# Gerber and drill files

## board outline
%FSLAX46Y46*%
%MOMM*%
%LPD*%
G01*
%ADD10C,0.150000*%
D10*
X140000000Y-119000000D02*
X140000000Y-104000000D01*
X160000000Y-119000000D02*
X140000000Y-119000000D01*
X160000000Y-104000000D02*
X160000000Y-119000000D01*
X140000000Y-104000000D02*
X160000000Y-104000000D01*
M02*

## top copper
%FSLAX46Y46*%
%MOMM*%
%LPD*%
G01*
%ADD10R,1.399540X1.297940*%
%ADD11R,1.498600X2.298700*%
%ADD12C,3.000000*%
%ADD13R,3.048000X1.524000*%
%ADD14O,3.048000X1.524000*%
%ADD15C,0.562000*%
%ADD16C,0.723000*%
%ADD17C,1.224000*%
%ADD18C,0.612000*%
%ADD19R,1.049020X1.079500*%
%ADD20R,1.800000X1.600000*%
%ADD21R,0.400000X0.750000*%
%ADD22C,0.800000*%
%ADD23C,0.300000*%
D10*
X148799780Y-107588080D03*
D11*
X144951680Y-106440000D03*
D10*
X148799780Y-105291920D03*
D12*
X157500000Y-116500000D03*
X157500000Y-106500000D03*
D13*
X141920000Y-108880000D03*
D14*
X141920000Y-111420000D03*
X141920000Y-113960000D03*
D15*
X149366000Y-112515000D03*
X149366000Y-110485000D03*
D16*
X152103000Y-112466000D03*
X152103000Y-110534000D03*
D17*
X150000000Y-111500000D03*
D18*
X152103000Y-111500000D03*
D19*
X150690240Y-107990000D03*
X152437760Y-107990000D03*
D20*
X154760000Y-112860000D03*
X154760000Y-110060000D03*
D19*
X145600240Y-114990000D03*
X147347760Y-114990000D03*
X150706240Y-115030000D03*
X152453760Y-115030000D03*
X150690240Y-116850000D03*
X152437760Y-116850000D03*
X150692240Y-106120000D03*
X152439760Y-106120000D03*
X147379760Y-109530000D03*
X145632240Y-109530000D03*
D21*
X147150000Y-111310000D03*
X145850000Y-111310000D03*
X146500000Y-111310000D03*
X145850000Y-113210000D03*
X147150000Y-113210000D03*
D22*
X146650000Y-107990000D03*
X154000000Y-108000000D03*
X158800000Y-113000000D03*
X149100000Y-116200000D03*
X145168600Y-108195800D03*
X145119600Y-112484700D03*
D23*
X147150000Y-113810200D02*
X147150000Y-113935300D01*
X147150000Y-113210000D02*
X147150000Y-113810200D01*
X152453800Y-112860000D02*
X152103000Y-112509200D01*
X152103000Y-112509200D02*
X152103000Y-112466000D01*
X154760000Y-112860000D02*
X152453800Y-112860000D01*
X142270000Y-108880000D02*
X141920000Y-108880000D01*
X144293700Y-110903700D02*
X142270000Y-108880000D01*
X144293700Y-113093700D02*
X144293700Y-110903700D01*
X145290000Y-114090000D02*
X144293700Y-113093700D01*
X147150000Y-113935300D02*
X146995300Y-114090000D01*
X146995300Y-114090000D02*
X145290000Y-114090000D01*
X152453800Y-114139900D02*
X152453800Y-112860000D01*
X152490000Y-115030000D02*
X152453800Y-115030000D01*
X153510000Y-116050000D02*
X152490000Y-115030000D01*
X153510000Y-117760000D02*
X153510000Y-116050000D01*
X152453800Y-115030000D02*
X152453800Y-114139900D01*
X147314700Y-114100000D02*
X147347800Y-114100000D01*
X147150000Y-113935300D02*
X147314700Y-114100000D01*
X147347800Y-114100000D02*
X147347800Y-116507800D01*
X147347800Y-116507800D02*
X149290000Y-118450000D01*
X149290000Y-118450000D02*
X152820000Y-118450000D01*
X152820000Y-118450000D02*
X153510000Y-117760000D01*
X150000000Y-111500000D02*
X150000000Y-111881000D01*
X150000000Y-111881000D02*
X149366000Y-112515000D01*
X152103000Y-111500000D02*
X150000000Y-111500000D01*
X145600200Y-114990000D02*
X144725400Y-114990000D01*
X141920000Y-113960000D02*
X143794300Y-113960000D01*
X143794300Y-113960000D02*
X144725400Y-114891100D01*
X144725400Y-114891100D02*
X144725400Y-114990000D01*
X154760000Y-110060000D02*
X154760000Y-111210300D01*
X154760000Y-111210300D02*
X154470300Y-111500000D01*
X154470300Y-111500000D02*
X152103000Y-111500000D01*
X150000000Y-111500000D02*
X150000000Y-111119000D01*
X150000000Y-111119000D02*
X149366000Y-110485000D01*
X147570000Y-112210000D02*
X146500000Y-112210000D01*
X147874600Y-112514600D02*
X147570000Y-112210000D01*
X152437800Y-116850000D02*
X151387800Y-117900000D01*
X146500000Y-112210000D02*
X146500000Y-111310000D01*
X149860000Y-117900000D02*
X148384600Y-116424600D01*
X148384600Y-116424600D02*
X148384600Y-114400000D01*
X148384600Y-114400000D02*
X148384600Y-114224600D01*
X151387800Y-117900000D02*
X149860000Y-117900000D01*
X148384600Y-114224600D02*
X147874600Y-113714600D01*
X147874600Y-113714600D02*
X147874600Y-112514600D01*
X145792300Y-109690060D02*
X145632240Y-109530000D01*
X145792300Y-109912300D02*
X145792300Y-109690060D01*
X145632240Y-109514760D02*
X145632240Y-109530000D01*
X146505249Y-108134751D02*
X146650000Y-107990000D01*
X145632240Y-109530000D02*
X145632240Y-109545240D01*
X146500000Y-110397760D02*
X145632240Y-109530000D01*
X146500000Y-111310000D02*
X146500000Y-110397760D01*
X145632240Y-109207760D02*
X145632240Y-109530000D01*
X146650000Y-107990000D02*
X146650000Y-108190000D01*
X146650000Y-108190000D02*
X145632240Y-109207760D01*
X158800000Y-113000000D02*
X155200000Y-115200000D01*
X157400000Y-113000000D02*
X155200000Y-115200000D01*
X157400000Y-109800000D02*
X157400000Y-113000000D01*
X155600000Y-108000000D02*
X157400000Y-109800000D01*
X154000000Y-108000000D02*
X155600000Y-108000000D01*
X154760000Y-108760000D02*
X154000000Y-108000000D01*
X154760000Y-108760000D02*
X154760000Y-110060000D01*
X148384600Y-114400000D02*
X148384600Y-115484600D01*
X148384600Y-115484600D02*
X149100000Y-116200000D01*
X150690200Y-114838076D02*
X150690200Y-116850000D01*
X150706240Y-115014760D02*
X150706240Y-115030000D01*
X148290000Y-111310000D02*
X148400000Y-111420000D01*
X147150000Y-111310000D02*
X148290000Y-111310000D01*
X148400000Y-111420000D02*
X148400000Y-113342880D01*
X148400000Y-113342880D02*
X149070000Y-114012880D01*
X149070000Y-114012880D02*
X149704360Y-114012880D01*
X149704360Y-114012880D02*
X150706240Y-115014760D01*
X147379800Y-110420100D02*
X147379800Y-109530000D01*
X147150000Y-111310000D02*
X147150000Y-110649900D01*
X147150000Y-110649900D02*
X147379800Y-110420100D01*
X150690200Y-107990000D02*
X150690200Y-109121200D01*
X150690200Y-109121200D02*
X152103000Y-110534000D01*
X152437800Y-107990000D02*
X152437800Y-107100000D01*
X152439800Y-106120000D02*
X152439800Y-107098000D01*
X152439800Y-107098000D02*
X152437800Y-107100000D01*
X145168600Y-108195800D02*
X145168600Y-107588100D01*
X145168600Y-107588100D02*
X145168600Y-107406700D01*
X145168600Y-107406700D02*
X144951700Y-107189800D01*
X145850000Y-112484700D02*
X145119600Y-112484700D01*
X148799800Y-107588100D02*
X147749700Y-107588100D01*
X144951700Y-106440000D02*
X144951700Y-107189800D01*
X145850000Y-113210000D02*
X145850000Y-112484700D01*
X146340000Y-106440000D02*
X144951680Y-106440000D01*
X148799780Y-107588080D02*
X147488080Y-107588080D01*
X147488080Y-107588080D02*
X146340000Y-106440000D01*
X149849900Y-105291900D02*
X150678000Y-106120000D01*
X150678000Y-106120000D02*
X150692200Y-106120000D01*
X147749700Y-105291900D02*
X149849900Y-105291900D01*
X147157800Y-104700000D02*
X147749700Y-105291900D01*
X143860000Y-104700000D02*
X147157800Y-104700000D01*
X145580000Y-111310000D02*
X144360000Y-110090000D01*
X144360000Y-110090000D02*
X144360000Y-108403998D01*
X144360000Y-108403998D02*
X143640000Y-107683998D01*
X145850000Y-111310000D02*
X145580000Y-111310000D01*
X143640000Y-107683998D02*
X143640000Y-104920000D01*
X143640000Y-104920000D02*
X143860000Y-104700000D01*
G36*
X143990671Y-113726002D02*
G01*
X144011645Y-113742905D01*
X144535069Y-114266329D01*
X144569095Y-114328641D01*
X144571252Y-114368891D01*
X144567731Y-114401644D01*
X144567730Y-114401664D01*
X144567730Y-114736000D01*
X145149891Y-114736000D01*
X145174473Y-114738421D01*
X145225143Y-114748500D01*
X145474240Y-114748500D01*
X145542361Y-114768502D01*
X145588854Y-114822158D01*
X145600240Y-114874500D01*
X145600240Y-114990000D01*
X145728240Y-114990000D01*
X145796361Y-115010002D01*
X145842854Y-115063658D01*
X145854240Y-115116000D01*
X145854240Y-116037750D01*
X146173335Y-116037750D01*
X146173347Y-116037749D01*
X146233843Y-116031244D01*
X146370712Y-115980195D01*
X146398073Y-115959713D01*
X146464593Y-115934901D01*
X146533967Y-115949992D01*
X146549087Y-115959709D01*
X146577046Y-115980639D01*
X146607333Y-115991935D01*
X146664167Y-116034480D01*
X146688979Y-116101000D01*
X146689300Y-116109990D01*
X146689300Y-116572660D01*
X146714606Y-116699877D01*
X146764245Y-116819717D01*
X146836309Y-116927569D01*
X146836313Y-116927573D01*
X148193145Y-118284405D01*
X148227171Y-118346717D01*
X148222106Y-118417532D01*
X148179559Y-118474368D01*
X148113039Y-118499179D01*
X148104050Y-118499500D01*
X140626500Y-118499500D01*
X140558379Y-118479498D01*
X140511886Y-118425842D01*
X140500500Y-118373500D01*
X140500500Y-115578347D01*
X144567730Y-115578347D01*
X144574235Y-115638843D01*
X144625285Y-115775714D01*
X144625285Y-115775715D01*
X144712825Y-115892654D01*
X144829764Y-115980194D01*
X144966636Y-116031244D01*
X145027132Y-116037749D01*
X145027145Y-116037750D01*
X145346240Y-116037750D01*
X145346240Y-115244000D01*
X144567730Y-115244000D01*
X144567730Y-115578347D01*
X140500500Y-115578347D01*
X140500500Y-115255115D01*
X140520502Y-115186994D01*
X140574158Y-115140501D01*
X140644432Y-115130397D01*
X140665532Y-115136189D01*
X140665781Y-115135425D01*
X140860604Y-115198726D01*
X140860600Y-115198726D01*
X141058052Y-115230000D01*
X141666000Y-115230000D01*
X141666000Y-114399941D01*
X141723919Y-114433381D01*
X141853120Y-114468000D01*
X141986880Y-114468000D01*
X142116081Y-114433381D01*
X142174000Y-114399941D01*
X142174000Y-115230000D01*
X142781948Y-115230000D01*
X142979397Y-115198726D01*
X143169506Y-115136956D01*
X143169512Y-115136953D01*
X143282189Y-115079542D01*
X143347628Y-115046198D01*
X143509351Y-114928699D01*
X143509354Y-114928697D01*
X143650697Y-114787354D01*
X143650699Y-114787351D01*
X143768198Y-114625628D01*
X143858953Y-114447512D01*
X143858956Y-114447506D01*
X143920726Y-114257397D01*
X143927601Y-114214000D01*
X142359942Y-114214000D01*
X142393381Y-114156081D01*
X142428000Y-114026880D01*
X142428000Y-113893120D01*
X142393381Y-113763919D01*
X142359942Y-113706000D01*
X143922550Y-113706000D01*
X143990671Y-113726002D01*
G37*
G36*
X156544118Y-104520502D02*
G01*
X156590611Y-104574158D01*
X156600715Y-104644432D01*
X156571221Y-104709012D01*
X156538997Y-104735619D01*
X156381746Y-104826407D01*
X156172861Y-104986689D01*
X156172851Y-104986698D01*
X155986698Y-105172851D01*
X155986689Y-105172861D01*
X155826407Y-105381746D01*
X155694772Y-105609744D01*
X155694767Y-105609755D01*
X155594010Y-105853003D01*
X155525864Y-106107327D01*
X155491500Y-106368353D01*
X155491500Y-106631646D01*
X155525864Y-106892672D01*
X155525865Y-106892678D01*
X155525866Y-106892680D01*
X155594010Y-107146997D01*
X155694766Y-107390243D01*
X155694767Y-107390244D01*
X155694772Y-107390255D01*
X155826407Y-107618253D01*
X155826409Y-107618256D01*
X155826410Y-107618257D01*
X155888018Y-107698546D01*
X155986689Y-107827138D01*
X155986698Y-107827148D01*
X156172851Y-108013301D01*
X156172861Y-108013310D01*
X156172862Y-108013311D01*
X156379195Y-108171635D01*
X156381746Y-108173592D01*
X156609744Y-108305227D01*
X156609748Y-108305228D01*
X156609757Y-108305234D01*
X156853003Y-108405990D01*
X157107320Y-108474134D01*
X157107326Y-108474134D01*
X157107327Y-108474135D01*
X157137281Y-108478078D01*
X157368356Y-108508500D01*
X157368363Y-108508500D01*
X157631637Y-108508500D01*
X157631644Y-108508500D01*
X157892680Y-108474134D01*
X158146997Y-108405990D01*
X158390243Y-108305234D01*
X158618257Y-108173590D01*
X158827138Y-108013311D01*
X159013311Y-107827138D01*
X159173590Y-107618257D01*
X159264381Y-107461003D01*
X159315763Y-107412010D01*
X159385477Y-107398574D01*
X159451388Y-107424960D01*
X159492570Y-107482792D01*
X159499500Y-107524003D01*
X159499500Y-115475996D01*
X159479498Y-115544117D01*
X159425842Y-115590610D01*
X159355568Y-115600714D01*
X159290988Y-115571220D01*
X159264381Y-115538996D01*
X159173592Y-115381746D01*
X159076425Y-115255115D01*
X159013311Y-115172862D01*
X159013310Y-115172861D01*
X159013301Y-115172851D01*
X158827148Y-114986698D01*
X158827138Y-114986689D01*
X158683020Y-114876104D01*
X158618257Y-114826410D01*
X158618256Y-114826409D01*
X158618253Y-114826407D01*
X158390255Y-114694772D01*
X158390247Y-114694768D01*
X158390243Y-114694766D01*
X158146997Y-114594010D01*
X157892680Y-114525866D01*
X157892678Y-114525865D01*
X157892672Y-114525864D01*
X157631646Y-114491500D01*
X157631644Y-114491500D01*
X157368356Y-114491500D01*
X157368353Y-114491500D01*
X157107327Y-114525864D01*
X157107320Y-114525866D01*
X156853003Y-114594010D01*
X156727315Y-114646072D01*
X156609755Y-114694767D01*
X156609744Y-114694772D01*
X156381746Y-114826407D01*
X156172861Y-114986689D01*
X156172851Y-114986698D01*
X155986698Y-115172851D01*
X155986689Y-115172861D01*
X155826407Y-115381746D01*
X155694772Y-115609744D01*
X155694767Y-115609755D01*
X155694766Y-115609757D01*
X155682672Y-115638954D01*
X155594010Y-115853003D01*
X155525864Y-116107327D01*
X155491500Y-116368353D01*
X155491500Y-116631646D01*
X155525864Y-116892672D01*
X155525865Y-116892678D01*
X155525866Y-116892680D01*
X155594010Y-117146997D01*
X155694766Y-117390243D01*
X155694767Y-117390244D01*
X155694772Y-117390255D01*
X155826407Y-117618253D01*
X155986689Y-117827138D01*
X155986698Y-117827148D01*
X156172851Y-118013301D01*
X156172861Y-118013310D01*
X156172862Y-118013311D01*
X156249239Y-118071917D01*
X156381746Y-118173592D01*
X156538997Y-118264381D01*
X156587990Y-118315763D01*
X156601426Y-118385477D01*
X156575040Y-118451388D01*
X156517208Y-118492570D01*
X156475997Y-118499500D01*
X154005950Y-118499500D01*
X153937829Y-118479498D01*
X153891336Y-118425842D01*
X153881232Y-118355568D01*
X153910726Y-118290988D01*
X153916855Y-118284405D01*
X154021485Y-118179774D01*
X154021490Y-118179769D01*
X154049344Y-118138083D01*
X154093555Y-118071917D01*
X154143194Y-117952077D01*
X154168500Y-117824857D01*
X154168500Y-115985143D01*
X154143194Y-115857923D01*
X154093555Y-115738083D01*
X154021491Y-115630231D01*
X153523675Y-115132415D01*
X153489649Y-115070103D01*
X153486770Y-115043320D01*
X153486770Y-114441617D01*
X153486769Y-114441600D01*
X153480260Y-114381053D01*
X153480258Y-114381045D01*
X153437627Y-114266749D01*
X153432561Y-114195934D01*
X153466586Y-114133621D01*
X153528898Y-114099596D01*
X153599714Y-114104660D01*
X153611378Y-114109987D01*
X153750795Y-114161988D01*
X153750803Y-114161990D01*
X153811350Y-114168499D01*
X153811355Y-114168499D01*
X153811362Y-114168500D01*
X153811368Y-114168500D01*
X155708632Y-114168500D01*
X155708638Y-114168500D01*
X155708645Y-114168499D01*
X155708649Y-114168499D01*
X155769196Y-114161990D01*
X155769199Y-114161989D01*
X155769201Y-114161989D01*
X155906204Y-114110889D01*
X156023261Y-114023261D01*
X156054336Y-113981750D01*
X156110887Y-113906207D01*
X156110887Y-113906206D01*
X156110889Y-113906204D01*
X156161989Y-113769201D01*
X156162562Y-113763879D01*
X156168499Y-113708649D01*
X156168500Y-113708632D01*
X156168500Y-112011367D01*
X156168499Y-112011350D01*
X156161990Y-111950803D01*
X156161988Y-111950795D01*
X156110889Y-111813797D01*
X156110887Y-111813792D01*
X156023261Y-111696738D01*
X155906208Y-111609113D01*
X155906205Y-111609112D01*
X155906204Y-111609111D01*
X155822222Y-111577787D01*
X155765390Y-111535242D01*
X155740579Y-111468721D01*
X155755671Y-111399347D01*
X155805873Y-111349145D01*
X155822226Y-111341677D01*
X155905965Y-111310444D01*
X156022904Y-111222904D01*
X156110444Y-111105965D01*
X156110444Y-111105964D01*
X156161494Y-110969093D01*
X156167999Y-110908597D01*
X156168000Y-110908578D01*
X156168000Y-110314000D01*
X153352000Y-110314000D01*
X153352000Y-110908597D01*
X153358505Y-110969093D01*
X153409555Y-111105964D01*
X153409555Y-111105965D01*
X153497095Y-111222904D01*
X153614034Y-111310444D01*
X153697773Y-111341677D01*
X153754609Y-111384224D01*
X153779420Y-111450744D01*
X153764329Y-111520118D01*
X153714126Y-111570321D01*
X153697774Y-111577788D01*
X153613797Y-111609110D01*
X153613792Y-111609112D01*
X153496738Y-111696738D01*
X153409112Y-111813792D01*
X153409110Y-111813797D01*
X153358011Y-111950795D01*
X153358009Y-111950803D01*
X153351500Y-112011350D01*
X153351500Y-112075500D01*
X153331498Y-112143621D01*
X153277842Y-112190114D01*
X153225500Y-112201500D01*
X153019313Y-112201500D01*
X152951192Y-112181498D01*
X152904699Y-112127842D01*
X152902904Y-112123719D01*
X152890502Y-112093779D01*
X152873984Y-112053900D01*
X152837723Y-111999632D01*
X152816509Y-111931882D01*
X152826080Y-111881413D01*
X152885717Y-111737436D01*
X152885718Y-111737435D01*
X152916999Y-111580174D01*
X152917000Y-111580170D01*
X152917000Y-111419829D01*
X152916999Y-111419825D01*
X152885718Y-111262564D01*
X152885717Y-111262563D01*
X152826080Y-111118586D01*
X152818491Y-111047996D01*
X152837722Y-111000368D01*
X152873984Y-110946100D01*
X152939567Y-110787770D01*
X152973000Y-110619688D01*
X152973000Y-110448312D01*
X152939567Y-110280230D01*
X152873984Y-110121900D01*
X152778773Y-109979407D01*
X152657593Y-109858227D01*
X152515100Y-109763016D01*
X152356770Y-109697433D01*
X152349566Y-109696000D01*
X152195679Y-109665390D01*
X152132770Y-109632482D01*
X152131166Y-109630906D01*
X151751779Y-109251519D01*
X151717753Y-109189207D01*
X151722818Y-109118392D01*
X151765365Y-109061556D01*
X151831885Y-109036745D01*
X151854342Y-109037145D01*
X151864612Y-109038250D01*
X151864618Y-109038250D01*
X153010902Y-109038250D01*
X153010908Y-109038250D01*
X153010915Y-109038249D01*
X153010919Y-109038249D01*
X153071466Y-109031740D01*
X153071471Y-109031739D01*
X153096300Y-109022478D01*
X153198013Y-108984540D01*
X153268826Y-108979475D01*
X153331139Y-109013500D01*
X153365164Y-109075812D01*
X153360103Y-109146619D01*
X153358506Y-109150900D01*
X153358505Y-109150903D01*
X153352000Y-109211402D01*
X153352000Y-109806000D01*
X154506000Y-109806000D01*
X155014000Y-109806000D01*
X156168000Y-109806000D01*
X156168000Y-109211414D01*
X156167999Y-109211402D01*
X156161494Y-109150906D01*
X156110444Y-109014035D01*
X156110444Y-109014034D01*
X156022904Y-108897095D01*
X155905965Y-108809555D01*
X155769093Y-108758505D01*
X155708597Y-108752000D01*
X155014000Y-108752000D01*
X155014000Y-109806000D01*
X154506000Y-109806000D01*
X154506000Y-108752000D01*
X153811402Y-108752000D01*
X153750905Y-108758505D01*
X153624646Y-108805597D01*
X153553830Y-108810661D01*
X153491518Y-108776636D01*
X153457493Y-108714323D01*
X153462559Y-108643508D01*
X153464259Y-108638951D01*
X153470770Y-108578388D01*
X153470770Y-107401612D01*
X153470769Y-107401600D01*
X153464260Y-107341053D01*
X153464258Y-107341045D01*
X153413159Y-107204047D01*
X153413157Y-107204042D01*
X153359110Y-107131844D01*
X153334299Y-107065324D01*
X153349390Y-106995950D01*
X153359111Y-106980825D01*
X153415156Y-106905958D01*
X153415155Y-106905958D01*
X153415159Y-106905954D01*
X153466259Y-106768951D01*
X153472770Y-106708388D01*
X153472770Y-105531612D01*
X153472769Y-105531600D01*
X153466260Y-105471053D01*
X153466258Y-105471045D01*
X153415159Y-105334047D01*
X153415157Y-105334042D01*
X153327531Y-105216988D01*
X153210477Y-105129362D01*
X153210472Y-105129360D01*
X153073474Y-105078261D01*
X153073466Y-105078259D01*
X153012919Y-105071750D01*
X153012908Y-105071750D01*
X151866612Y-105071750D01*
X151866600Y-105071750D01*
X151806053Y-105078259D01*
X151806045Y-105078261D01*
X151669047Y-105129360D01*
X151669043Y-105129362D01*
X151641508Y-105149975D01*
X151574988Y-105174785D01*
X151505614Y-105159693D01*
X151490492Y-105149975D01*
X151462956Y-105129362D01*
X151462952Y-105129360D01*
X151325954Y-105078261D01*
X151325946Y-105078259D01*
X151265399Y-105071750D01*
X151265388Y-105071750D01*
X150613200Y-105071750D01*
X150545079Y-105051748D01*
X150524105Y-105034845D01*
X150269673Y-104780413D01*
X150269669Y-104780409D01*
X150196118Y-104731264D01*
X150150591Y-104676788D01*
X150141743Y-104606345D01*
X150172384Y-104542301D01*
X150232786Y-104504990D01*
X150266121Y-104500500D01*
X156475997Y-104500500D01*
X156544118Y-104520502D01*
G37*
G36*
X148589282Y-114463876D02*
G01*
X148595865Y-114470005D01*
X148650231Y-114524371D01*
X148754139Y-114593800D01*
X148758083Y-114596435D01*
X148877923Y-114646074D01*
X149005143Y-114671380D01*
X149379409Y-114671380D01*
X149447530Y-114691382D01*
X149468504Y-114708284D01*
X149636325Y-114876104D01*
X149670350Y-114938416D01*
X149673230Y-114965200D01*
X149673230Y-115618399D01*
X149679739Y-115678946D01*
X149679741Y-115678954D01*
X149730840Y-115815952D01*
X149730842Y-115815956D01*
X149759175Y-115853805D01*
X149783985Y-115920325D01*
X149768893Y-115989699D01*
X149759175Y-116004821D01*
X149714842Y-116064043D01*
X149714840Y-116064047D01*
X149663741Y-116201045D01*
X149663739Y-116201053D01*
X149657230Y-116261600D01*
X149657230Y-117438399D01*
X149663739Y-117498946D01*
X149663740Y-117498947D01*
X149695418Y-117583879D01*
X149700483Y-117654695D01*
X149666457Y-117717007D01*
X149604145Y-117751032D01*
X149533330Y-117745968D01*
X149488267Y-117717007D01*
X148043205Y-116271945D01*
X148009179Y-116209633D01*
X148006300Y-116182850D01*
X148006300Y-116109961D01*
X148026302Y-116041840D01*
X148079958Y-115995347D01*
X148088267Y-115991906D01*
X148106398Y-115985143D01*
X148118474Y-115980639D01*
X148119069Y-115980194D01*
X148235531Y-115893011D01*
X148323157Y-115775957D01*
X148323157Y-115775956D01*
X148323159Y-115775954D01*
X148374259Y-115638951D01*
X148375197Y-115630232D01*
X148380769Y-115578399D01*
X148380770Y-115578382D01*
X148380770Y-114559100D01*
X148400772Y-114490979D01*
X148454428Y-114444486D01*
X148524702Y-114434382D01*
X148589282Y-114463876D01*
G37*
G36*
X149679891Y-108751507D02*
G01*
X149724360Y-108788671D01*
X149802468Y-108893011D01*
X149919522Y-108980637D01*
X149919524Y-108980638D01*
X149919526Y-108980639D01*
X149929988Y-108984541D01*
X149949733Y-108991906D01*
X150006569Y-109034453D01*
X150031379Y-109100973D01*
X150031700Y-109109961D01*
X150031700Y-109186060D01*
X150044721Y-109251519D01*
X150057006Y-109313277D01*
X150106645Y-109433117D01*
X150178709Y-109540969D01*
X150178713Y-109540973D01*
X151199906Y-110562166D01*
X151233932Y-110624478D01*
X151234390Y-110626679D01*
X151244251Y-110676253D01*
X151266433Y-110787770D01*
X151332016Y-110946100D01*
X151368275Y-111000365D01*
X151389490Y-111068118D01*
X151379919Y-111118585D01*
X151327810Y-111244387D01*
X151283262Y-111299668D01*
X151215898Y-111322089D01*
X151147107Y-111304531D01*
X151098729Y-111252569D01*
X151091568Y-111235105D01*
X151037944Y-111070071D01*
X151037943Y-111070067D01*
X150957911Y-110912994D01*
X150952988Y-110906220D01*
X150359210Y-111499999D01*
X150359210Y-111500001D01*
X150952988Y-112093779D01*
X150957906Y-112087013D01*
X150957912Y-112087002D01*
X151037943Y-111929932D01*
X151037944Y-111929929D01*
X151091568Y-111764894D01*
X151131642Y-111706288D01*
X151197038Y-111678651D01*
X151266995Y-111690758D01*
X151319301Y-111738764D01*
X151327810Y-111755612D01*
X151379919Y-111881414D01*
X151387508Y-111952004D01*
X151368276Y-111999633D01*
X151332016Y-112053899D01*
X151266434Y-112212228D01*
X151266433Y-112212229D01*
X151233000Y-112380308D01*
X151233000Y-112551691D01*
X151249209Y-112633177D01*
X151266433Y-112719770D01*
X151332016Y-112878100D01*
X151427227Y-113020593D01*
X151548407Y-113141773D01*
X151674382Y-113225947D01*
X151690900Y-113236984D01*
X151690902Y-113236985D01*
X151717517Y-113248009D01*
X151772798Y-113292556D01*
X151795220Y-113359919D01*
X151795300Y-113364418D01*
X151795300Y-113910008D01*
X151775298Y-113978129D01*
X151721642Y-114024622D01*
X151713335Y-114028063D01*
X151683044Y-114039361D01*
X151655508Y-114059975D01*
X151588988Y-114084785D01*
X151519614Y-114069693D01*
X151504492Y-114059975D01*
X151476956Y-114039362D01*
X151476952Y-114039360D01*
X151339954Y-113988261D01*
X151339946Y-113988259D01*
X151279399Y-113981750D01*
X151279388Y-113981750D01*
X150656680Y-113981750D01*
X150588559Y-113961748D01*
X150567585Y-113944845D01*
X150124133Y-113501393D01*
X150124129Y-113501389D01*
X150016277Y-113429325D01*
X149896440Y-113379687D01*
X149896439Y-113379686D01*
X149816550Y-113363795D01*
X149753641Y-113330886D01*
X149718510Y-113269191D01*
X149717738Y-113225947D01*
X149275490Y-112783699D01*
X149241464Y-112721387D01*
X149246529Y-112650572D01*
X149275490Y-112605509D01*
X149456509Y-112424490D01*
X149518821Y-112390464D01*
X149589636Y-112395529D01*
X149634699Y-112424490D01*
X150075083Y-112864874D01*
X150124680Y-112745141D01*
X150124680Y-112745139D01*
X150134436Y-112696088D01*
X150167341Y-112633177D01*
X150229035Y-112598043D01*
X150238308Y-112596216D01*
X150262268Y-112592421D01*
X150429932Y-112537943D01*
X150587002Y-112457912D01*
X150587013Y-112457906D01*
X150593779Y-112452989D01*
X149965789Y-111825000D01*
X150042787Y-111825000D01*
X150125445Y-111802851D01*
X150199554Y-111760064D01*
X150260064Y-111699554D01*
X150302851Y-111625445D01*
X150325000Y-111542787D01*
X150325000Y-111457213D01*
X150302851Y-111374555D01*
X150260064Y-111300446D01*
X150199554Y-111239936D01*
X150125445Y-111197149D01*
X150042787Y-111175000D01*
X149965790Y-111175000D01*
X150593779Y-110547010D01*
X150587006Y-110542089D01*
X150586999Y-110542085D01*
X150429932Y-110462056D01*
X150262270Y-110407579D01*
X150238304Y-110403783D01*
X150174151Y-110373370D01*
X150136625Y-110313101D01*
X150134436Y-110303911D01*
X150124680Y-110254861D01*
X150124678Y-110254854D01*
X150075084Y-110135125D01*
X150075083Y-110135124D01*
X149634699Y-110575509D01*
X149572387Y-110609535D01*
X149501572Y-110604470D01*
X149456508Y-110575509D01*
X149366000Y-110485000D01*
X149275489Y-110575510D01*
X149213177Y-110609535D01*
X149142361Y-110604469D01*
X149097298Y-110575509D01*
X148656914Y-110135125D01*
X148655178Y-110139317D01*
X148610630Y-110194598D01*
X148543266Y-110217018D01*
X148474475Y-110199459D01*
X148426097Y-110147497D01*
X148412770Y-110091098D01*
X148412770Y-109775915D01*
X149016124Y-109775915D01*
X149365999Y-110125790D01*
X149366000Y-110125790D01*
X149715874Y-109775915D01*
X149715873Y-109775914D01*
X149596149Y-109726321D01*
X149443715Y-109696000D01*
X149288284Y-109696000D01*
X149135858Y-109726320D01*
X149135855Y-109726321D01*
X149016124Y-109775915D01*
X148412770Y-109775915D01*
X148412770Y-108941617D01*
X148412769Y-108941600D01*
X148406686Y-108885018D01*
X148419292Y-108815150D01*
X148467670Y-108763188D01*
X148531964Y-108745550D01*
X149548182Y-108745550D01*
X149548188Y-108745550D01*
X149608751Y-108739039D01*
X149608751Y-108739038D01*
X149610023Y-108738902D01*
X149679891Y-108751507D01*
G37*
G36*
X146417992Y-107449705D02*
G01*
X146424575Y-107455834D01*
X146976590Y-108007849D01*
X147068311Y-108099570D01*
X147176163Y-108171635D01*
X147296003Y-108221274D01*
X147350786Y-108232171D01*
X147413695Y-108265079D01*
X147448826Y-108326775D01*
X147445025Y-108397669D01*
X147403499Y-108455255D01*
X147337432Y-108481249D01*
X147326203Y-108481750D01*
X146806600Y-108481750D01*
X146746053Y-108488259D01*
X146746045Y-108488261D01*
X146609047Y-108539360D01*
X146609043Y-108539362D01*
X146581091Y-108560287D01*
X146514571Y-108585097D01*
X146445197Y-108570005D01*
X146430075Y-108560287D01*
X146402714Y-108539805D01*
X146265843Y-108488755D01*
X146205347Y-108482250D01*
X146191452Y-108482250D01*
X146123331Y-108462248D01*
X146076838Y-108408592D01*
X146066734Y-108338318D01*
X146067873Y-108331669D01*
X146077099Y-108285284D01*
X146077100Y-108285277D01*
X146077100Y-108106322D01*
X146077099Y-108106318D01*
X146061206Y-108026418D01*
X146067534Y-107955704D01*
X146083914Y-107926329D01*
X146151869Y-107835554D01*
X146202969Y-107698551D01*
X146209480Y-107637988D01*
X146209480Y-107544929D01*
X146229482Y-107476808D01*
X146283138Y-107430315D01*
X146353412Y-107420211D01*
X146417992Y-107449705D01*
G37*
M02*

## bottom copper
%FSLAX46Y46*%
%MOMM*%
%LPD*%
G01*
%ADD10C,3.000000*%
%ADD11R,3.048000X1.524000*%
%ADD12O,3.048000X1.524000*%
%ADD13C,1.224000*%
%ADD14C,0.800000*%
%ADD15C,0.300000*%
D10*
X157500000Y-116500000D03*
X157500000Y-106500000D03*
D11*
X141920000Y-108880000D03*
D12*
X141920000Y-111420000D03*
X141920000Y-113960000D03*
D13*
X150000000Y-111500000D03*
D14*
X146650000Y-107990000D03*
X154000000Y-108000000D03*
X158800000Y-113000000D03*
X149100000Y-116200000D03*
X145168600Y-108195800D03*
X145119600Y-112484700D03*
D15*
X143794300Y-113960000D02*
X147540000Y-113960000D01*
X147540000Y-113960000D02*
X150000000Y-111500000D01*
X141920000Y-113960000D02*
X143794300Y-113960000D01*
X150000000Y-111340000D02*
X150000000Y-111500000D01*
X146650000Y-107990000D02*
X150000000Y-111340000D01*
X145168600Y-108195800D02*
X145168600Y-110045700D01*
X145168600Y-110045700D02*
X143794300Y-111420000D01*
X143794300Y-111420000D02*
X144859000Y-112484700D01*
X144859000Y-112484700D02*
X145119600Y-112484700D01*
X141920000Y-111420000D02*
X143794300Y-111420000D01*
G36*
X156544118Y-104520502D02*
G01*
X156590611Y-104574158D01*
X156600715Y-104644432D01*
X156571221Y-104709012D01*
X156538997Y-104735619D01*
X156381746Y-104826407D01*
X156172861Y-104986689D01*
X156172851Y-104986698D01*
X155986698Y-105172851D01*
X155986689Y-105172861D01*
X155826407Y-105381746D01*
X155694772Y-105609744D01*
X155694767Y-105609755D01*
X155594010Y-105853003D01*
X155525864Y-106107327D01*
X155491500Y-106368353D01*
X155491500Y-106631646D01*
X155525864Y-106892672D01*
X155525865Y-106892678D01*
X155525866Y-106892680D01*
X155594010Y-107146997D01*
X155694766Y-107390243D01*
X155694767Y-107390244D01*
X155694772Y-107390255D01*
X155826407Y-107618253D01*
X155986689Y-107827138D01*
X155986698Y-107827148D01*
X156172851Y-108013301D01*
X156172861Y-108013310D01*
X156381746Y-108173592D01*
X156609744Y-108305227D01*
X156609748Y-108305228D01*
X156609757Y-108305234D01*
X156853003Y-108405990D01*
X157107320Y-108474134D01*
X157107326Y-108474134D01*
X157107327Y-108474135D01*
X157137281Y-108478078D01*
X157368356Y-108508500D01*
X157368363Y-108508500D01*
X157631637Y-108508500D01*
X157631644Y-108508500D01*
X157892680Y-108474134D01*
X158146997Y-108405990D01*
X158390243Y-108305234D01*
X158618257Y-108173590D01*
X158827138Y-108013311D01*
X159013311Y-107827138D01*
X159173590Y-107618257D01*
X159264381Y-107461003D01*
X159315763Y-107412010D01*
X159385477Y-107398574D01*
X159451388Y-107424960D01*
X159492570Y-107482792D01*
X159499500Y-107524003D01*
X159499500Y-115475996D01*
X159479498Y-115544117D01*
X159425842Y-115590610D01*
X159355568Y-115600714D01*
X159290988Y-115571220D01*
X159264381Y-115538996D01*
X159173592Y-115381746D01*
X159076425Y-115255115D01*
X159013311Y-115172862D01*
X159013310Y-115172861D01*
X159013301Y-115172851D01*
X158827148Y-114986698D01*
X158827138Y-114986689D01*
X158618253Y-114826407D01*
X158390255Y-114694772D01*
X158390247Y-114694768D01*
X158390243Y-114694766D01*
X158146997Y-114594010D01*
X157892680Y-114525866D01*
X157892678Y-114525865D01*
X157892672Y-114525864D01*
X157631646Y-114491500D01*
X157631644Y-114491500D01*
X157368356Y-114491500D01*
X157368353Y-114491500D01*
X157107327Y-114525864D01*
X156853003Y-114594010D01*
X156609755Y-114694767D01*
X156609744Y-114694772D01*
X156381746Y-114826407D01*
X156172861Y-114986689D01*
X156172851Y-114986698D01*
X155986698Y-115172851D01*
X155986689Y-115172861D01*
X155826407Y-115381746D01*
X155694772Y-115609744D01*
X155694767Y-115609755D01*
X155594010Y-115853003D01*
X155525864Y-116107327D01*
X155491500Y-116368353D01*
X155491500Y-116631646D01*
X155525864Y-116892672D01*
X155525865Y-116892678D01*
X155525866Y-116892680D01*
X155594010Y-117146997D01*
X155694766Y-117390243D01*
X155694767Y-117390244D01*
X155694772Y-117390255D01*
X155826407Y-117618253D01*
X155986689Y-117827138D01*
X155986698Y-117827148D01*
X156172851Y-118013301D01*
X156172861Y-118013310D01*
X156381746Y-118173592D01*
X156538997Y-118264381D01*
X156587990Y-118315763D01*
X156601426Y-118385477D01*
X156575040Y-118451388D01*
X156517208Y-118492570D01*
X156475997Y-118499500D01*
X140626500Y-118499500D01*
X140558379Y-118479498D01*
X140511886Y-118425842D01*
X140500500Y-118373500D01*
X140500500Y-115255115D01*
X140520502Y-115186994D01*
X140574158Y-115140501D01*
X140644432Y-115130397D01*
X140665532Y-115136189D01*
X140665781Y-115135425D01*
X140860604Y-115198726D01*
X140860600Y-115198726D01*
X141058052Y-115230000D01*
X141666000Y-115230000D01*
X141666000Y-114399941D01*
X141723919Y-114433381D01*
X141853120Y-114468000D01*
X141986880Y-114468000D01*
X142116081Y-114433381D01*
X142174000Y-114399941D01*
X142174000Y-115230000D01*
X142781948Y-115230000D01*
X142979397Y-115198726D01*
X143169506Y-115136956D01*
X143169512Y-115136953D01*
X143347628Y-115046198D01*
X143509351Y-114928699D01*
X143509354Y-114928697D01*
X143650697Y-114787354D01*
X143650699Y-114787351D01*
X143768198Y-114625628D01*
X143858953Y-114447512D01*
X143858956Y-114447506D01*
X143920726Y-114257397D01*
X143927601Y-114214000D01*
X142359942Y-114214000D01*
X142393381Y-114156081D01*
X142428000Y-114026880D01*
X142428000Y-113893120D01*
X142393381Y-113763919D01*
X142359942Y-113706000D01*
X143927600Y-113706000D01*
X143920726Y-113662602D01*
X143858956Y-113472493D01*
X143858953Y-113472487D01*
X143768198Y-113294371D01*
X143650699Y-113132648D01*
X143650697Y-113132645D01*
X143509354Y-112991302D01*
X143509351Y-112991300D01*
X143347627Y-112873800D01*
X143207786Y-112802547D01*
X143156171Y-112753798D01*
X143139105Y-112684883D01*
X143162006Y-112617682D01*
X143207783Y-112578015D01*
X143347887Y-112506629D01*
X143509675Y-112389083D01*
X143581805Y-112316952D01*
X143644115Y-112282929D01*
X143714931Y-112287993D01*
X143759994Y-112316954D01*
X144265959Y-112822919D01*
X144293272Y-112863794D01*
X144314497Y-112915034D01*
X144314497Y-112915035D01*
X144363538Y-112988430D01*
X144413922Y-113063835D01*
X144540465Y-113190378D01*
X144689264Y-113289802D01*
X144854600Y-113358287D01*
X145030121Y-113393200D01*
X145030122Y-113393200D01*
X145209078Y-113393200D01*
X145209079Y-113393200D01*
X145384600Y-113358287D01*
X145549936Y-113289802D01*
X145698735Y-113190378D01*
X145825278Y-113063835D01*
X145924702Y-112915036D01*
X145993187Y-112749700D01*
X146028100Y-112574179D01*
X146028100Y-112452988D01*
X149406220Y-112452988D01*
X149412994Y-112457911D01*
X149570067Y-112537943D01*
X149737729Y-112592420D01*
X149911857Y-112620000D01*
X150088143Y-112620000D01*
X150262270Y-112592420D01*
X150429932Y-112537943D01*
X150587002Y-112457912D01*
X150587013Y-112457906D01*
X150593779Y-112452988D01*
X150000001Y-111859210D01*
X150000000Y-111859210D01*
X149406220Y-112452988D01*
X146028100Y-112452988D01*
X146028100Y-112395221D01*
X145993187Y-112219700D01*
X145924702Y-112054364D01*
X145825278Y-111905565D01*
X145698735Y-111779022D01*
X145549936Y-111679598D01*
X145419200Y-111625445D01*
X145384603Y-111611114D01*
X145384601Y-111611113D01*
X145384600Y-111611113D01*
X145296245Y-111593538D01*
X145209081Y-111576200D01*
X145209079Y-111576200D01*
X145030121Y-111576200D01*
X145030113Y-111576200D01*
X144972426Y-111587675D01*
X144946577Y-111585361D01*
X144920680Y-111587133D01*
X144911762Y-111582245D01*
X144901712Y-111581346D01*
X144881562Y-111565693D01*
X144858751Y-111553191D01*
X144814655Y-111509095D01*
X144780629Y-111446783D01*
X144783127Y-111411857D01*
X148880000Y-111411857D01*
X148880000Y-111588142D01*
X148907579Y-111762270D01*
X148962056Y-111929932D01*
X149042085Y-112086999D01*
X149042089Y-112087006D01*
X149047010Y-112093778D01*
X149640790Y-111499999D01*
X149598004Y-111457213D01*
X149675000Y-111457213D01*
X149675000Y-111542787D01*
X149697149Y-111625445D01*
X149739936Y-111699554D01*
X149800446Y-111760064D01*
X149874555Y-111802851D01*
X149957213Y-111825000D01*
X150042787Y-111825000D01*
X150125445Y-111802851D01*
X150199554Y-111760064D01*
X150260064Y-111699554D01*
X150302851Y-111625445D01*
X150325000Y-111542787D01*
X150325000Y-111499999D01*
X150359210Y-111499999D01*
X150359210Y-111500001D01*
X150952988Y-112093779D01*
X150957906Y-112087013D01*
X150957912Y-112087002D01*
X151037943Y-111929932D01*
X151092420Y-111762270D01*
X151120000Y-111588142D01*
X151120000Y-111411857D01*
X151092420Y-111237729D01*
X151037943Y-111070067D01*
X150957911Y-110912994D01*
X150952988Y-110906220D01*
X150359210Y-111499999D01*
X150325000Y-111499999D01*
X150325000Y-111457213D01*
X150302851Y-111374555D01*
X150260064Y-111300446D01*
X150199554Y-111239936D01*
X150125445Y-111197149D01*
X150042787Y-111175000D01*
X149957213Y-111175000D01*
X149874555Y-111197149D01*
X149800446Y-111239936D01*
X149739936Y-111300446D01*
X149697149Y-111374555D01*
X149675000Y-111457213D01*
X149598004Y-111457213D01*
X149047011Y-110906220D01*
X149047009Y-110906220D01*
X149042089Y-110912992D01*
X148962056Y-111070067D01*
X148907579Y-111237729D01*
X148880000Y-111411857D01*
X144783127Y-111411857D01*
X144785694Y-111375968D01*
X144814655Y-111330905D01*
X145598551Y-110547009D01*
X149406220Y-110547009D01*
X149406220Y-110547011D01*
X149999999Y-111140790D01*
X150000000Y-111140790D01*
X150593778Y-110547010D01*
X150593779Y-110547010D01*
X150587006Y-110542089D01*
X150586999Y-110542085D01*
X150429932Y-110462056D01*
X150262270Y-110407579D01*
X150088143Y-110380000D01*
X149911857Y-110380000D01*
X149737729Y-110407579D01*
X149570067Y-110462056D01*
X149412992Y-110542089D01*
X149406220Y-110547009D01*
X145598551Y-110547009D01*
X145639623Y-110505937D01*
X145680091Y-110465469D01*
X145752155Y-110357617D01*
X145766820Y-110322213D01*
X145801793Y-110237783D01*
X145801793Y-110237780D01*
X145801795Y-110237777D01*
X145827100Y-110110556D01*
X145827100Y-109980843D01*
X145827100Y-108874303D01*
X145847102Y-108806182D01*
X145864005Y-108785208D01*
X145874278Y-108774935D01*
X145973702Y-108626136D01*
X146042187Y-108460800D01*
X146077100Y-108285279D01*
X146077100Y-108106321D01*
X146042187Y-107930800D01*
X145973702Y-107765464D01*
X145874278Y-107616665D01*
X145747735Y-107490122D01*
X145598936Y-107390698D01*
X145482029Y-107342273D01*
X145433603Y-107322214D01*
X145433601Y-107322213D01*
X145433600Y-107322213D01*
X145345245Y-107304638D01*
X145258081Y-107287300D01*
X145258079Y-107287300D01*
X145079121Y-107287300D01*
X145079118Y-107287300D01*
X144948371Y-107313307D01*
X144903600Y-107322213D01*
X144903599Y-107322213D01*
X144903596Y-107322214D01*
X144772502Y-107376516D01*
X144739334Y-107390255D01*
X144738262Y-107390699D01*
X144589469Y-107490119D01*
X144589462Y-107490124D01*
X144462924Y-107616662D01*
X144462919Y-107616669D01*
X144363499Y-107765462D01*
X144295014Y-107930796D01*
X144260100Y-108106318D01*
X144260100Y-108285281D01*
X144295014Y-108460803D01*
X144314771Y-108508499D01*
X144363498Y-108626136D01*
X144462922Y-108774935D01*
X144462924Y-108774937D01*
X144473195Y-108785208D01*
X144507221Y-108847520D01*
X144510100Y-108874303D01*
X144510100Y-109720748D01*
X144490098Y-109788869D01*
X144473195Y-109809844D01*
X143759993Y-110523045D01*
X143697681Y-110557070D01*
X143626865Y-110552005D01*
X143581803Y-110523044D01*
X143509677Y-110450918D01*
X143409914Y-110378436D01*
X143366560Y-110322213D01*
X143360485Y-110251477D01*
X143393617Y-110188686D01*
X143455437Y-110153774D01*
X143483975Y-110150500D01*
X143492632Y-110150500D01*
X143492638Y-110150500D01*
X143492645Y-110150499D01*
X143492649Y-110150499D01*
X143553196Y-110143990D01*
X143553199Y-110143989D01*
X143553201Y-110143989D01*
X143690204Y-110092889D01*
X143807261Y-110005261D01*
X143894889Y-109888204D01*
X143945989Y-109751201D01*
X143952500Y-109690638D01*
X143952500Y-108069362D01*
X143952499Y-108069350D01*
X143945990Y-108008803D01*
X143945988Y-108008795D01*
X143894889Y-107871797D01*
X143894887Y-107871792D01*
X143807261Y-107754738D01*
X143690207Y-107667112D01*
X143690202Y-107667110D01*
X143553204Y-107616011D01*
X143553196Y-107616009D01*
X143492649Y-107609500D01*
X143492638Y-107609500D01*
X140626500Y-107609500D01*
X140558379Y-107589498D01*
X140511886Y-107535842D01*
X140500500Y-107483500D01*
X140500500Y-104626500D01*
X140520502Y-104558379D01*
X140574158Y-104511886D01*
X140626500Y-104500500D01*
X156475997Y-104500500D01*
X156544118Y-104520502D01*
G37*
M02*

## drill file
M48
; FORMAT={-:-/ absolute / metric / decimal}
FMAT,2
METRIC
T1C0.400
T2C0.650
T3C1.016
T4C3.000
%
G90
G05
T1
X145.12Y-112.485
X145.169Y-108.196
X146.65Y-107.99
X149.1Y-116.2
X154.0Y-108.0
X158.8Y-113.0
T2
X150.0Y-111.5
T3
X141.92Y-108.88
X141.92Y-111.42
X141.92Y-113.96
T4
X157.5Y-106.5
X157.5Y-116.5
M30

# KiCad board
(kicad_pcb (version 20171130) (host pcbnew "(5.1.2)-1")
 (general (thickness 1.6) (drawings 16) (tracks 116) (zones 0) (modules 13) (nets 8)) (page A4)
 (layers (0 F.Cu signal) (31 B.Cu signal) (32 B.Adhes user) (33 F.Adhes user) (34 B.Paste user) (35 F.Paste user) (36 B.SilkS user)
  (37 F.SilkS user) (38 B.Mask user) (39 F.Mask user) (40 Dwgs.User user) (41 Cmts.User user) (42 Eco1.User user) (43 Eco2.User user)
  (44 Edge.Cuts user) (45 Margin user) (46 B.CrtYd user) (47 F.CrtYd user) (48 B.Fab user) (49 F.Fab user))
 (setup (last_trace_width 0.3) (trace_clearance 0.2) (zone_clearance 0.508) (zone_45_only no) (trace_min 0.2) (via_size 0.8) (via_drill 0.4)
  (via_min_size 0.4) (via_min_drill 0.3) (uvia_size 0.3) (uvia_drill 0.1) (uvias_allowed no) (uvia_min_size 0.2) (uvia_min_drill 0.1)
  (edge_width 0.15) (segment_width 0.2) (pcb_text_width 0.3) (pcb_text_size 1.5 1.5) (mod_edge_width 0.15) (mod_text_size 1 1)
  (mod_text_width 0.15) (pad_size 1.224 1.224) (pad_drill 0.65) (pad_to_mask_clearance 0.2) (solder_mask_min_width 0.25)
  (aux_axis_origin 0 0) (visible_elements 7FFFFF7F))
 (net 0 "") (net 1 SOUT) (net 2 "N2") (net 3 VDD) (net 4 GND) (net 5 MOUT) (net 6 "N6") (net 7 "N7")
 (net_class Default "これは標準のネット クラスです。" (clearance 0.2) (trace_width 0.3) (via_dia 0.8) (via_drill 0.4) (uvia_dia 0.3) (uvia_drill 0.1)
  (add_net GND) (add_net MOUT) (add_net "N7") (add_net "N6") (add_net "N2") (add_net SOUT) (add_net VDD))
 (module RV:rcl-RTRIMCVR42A (layer F.Cu) (at 146.75 106.44 90)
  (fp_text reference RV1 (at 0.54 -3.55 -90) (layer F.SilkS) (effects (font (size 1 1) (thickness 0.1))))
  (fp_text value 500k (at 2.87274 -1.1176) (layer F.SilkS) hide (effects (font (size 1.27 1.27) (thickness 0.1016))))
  (pad 1 smd rect (at -1.14808 2.04978 90) (size 1.29794 1.39954) (layers F.Cu F.Paste F.Mask) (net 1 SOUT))
  (pad 2 smd rect (at 0 -1.79832 90) (size 2.2987 1.4986) (layers F.Cu F.Paste F.Mask) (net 1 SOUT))
  (pad 3 smd rect (at 1.14808 2.04978 90) (size 1.29794 1.39954) (layers F.Cu F.Paste F.Mask) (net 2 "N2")))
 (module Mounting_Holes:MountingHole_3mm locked (layer F.Cu) (at 157.5 116.5)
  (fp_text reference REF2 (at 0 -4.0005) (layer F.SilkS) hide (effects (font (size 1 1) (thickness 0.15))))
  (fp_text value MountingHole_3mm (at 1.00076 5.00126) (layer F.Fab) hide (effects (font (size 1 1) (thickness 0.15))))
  (pad 1 thru_hole circle (at 0 0) (size 3 3) (drill 3) (layers)))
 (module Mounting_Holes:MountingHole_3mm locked (layer F.Cu) (at 157.5 106.5)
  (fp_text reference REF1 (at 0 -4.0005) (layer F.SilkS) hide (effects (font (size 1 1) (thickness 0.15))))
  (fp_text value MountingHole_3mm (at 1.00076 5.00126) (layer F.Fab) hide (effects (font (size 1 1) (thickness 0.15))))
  (pad 1 thru_hole circle (at 0 0) (size 3 3) (drill 3) (layers)))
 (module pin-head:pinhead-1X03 (layer F.Cu) (at 141.92 111.42 270)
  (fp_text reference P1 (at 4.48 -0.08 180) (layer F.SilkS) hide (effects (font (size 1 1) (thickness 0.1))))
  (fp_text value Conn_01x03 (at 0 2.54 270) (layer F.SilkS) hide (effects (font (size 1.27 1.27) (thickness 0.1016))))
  (pad 1 thru_hole rect (at -2.54 0 90) (size 1.524 3.048) (drill 1.016) (layers *.Cu *.Paste *.Mask F.SilkS) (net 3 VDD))
  (pad 2 thru_hole oval (at 0 0 90) (size 1.524 3.048) (drill 1.016) (layers *.Cu *.Paste *.Mask F.SilkS) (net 1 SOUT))
  (pad 3 thru_hole oval (at 2.54 0 90) (size 1.524 3.048) (drill 1.016) (layers *.Cu *.Paste *.Mask F.SilkS) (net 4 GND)))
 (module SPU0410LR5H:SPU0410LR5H (layer F.Cu) (at 150 111.5 270)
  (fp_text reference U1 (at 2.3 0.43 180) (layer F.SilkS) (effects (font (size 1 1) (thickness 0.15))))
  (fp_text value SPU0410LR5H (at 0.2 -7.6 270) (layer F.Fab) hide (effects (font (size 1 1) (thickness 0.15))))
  (pad 3 smd circle (at 1.015 0.634 270) (size 0.562 0.562) (layers F.Cu F.Paste F.Mask) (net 4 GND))
  (pad 2 smd circle (at -1.015 0.634 270) (size 0.562 0.562) (layers F.Cu F.Paste F.Mask) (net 4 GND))
  (pad 4 smd circle (at 0.966 -2.103 270) (size 0.723 0.723) (layers F.Cu F.Paste F.Mask) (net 3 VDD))
  (pad 1 smd circle (at -0.966 -2.103 270) (size 0.723 0.723) (layers F.Cu F.Paste F.Mask) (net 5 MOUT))
  (pad 6 thru_hole circle (at 0 0 270) (size 1.224 1.224) (drill 0.65) (layers *.Cu F.Paste F.Mask) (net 4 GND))
  (pad 5 smd circle (at 0 -2.103 270) (size 0.612 0.612) (layers F.Cu F.Paste F.Mask) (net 4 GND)))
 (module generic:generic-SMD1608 (layer F.Cu) (at 151.564 107.99 180)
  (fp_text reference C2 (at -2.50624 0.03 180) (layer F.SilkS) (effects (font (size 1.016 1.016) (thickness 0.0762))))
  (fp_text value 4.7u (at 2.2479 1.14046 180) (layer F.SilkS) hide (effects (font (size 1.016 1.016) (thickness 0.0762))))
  (pad 2 smd rect (at 0.87376 0 180) (size 1.04902 1.0795) (layers F.Cu F.Paste F.Mask) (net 5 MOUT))
  (pad 1 smd rect (at -0.87376 0 180) (size 1.04902 1.0795) (layers F.Cu F.Paste F.Mask) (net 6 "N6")))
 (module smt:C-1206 (layer F.Cu) (at 154.76 111.46 90)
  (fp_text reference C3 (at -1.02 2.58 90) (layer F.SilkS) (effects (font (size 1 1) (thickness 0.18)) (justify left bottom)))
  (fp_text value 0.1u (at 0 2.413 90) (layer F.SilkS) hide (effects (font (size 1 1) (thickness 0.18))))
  (pad 1 smd rect (at -1.4 0 90) (size 1.6 1.8) (layers F.Cu F.Paste F.Mask) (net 3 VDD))
  (pad 2 smd rect (at 1.4 0 90) (size 1.6 1.8) (layers F.Cu F.Paste F.Mask) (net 4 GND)))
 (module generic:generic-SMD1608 (layer F.Cu) (at 146.474 114.99 180)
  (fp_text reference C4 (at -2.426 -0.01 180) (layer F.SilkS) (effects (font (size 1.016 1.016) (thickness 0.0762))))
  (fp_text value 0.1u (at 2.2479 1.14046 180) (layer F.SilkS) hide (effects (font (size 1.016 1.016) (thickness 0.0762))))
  (pad 2 smd rect (at 0.87376 0 180) (size 1.04902 1.0795) (layers F.Cu F.Paste F.Mask) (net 4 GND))
  (pad 1 smd rect (at -0.87376 0 180) (size 1.04902 1.0795) (layers F.Cu F.Paste F.Mask) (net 3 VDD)))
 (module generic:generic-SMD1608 (layer F.Cu) (at 151.58 115.03)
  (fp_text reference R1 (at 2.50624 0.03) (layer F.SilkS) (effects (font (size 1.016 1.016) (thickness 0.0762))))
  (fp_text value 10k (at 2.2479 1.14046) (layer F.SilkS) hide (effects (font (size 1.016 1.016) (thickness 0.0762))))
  (pad 1 smd rect (at -0.87376 0) (size 1.04902 1.0795) (layers F.Cu F.Paste F.Mask) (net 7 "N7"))
  (pad 2 smd rect (at 0.87376 0) (size 1.04902 1.0795) (layers F.Cu F.Paste F.Mask) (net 3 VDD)))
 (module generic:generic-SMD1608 (layer F.Cu) (at 151.564 116.85 180)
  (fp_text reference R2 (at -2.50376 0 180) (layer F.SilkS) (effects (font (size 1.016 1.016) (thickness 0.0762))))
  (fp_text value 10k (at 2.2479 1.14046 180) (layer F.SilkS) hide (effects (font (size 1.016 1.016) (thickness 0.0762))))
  (pad 2 smd rect (at 0.87376 0 180) (size 1.04902 1.0795) (layers F.Cu F.Paste F.Mask) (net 7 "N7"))
  (pad 1 smd rect (at -0.87376 0 180) (size 1.04902 1.0795) (layers F.Cu F.Paste F.Mask) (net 4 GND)))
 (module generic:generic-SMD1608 (layer F.Cu) (at 151.566 106.12)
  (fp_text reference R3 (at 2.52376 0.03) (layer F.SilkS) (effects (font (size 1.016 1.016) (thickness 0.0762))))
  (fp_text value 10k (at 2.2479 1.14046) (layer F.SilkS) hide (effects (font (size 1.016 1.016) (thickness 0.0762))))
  (pad 1 smd rect (at -0.87376 0) (size 1.04902 1.0795) (layers F.Cu F.Paste F.Mask) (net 2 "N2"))
  (pad 2 smd rect (at 0.87376 0) (size 1.04902 1.0795) (layers F.Cu F.Paste F.Mask) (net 6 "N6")))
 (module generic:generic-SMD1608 (layer F.Cu) (at 146.506 109.53 180)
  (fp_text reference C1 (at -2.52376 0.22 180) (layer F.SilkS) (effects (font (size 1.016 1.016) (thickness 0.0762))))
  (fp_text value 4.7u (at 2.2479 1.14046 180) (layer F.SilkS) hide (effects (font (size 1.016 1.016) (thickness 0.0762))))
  (pad 1 smd rect (at -0.87376 0 180) (size 1.04902 1.0795) (layers F.Cu F.Paste F.Mask) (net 7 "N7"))
  (pad 2 smd rect (at 0.87376 0 180) (size 1.04902 1.0795) (layers F.Cu F.Paste F.Mask) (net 4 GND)))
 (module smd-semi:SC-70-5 (layer F.Cu) (at 146.5 112.26 270)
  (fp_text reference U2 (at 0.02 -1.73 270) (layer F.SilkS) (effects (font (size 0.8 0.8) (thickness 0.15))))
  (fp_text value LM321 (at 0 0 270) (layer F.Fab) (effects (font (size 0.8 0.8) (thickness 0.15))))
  (pad 1 smd rect (at -0.95 -0.65 90) (size 0.75 0.4) (layers F.Cu F.Paste F.Mask) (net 7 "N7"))
  (pad 3 smd rect (at -0.95 0.65 90) (size 0.75 0.4) (layers F.Cu F.Paste F.Mask) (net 2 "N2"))
  (pad 2 smd rect (at -0.95 0 90) (size 0.75 0.4) (layers F.Cu F.Paste F.Mask) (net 4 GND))
  (pad 4 smd rect (at 0.95 0.65 90) (size 0.75 0.4) (layers F.Cu F.Paste F.Mask) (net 1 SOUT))
  (pad 5 smd rect (at 0.95 -0.65 90) (size 0.75 0.4) (layers F.Cu F.Paste F.Mask) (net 3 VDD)))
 (gr_line (start 140 119) (end 140 104) (angle 90) (layer Edge.Cuts) (width 0.15))
 (gr_line (start 160 119) (end 140 119) (angle 90) (layer Edge.Cuts) (width 0.15))
 (gr_line (start 160 104) (end 160 119) (angle 90) (layer Edge.Cuts) (width 0.15))
 (gr_line (start 140 104) (end 160 104) (angle 90) (layer Edge.Cuts) (width 0.15))
 (segment (start 147.15 113.8102) (end 147.15 113.9353) (width 0.3) (layer F.Cu) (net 3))
 (segment (start 147.15 113.21) (end 147.15 113.8102) (width 0.3) (layer F.Cu) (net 3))
 (segment (start 152.4538 112.86) (end 152.103 112.5092) (width 0.3) (layer F.Cu) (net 3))
 (segment (start 152.103 112.5092) (end 152.103 112.466) (width 0.3) (layer F.Cu) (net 3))
 (segment (start 154.76 112.86) (end 152.4538 112.86) (width 0.3) (layer F.Cu) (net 3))
 (segment (start 142.27 108.88) (end 141.92 108.88) (width 0.3) (layer F.Cu) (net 3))
 (segment (start 144.2937 110.9037) (end 142.27 108.88) (width 0.3) (layer F.Cu) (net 3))
 (segment (start 144.2937 113.0937) (end 144.2937 110.9037) (width 0.3) (layer F.Cu) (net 3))
 (segment (start 145.29 114.09) (end 144.2937 113.0937) (width 0.3) (layer F.Cu) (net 3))
 (segment (start 147.15 113.9353) (end 146.9953 114.09) (width 0.3) (layer F.Cu) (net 3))
 (segment (start 146.9953 114.09) (end 145.29 114.09) (width 0.3) (layer F.Cu) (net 3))
 (segment (start 152.4538 114.1399) (end 152.4538 112.86) (width 0.3) (layer F.Cu) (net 3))
 (segment (start 152.49 115.03) (end 152.4538 115.03) (width 0.3) (layer F.Cu) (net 3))
 (segment (start 153.51 116.05) (end 152.49 115.03) (width 0.3) (layer F.Cu) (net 3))
 (segment (start 153.51 117.76) (end 153.51 116.05) (width 0.3) (layer F.Cu) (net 3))
 (segment (start 152.4538 115.03) (end 152.4538 114.1399) (width 0.3) (layer F.Cu) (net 3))
 (segment (start 147.3147 114.1) (end 147.3478 114.1) (width 0.3) (layer F.Cu) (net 3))
 (segment (start 147.15 113.9353) (end 147.3147 114.1) (width 0.3) (layer F.Cu) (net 3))
 (segment (start 147.3478 114.1) (end 147.3478 116.5078) (width 0.3) (layer F.Cu) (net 3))
 (segment (start 147.3478 116.5078) (end 149.29 118.45) (width 0.3) (layer F.Cu) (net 3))
 (segment (start 149.29 118.45) (end 152.82 118.45) (width 0.3) (layer F.Cu) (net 3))
 (segment (start 152.82 118.45) (end 153.51 117.76) (width 0.3) (layer F.Cu) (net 3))
 (segment (start 150 111.5) (end 150 111.881) (width 0.3) (layer F.Cu) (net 4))
 (segment (start 150 111.881) (end 149.366 112.515) (width 0.3) (layer F.Cu) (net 4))
 (segment (start 152.103 111.5) (end 150 111.5) (width 0.3) (layer F.Cu) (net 4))
 (segment (start 145.6002 114.99) (end 144.7254 114.99) (width 0.3) (layer F.Cu) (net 4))
 (segment (start 141.92 113.96) (end 143.7943 113.96) (width 0.3) (layer F.Cu) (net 4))
 (segment (start 143.7943 113.96) (end 144.7254 114.8911) (width 0.3) (layer F.Cu) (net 4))
 (segment (start 144.7254 114.8911) (end 144.7254 114.99) (width 0.3) (layer F.Cu) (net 4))
 (segment (start 154.76 110.06) (end 154.76 111.2103) (width 0.3) (layer F.Cu) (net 4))
 (segment (start 154.76 111.2103) (end 154.4703 111.5) (width 0.3) (layer F.Cu) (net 4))
 (segment (start 154.4703 111.5) (end 152.103 111.5) (width 0.3) (layer F.Cu) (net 4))
 (segment (start 150 111.5) (end 150 111.119) (width 0.3) (layer F.Cu) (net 4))
 (segment (start 150 111.119) (end 149.366 110.485) (width 0.3) (layer F.Cu) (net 4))
 (segment (start 143.7943 113.96) (end 147.54 113.96) (width 0.3) (layer B.Cu) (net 4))
 (segment (start 147.54 113.96) (end 150 111.5) (width 0.3) (layer B.Cu) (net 4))
 (segment (start 141.92 113.96) (end 143.7943 113.96) (width 0.3) (layer B.Cu) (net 4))
 (segment (start 147.57 112.21) (end 146.5 112.21) (width 0.3) (layer F.Cu) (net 4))
 (segment (start 147.8746 112.5146) (end 147.57 112.21) (width 0.3) (layer F.Cu) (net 4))
 (segment (start 152.4378 116.85) (end 151.3878 117.9) (width 0.3) (layer F.Cu) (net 4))
 (segment (start 146.5 112.21) (end 146.5 111.31) (width 0.3) (layer F.Cu) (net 4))
 (segment (start 149.86 117.9) (end 148.3846 116.4246) (width 0.3) (layer F.Cu) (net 4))
 (segment (start 148.3846 116.4246) (end 148.3846 114.4) (width 0.3) (layer F.Cu) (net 4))
 (segment (start 148.3846 114.4) (end 148.3846 114.2246) (width 0.3) (layer F.Cu) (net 4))
 (segment (start 151.3878 117.9) (end 149.86 117.9) (width 0.3) (layer F.Cu) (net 4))
 (segment (start 148.3846 114.2246) (end 147.8746 113.7146) (width 0.3) (layer F.Cu) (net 4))
 (segment (start 147.8746 113.7146) (end 147.8746 112.5146) (width 0.3) (layer F.Cu) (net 4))
 (segment (start 145.7923 109.69006) (end 145.63224 109.53) (width 0.3) (layer F.Cu) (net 4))
 (segment (start 145.7923 109.9123) (end 145.7923 109.69006) (width 0.3) (layer F.Cu) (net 4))
 (segment (start 145.63224 109.51476) (end 145.63224 109.53) (width 0.3) (layer F.Cu) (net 4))
 (segment (start 146.505249 108.134751) (end 146.65 107.99) (width 0.3) (layer F.Cu) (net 4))
 (via (at 146.65 107.99) (size 0.8) (drill 0.4) (layers F.Cu B.Cu) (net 4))
 (segment (start 145.63224 109.53) (end 145.63224 109.54524) (width 0.3) (layer F.Cu) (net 4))
 (segment (start 150 111.34) (end 150 111.5) (width 0.3) (layer B.Cu) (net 4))
 (segment (start 146.65 107.99) (end 150 111.34) (width 0.3) (layer B.Cu) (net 4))
 (segment (start 146.5 110.39776) (end 145.63224 109.53) (width 0.3) (layer F.Cu) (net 4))
 (segment (start 146.5 111.31) (end 146.5 110.39776) (width 0.3) (layer F.Cu) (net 4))
 (segment (start 145.63224 109.20776) (end 145.63224 109.53) (width 0.3) (layer F.Cu) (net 4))
 (segment (start 146.65 107.99) (end 146.65 108.19) (width 0.3) (layer F.Cu) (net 4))
 (segment (start 146.65 108.19) (end 145.63224 109.20776) (width 0.3) (layer F.Cu) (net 4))
 (via (at 154 108) (size 0.8) (drill 0.4) (layers F.Cu B.Cu) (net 4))
 (via (at 158.8 113) (size 0.8) (drill 0.4) (layers F.Cu B.Cu) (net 4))
 (segment (start 158.8 113) (end 155.2 115.2) (width 0.3) (layer F.Cu) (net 4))
 (segment (start 157.4 113) (end 155.2 115.2) (width 0.3) (layer F.Cu) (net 4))
 (segment (start 157.4 109.8) (end 157.4 113) (width 0.3) (layer F.Cu) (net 4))
 (segment (start 155.6 108) (end 157.4 109.8) (width 0.3) (layer F.Cu) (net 4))
 (segment (start 154 108) (end 155.6 108) (width 0.3) (layer F.Cu) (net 4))
 (segment (start 154.76 108.76) (end 154 108) (width 0.3) (layer F.Cu) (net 4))
 (segment (start 154.76 108.76) (end 154.76 110.06) (width 0.3) (layer F.Cu) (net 4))
 (segment (start 148.3846 114.4) (end 148.3846 115.4846) (width 0.3) (layer F.Cu) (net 4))
 (via (at 149.1 116.2) (size 0.8) (drill 0.4) (layers F.Cu B.Cu) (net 4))
 (segment (start 148.3846 115.4846) (end 149.1 116.2) (width 0.3) (layer F.Cu) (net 4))
 (segment (start 150.6902 114.838076) (end 150.6902 116.85) (width 0.3) (layer F.Cu) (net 7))
 (segment (start 150.70624 115.01476) (end 150.70624 115.03) (width 0.3) (layer F.Cu) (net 7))
 (segment (start 148.29 111.31) (end 148.4 111.42) (width 0.3) (layer F.Cu) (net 7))
 (segment (start 147.15 111.31) (end 148.29 111.31) (width 0.3) (layer F.Cu) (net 7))
 (segment (start 148.4 111.42) (end 148.4 113.34288) (width 0.3) (layer F.Cu) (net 7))
 (segment (start 148.4 113.34288) (end 149.07 114.01288) (width 0.3) (layer F.Cu) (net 7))
 (segment (start 149.07 114.01288) (end 149.70436 114.01288) (width 0.3) (layer F.Cu) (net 7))
 (segment (start 149.70436 114.01288) (end 150.70624 115.01476) (width 0.3) (layer F.Cu) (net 7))
 (segment (start 147.3798 110.4201) (end 147.3798 109.53) (width 0.3) (layer F.Cu) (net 7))
 (segment (start 147.15 111.31) (end 147.15 110.6499) (width 0.3) (layer F.Cu) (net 7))
 (segment (start 147.15 110.6499) (end 147.3798 110.4201) (width 0.3) (layer F.Cu) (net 7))
 (segment (start 150.6902 107.99) (end 150.6902 109.1212) (width 0.3) (layer F.Cu) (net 5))
 (segment (start 150.6902 109.1212) (end 152.103 110.534) (width 0.3) (layer F.Cu) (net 5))
 (segment (start 152.4378 107.99) (end 152.4378 107.1) (width 0.3) (layer F.Cu) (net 6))
 (segment (start 152.4398 106.12) (end 152.4398 107.098) (width 0.3) (layer F.Cu) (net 6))
 (segment (start 152.4398 107.098) (end 152.4378 107.1) (width 0.3) (layer F.Cu) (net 6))
 (segment (start 145.1686 108.1958) (end 145.1686 110.0457) (width 0.3) (layer B.Cu) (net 1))
 (segment (start 145.1686 110.0457) (end 143.7943 111.42) (width 0.3) (layer B.Cu) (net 1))
 (segment (start 145.1686 108.1958) (end 145.1686 107.5881) (width 0.3) (layer F.Cu) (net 1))
 (segment (start 143.7943 111.42) (end 144.859 112.4847) (width 0.3) (layer B.Cu) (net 1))
 (segment (start 144.859 112.4847) (end 145.1196 112.4847) (width 0.3) (layer B.Cu) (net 1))
 (segment (start 145.1686 107.5881) (end 145.1686 107.4067) (width 0.3) (layer F.Cu) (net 1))
 (segment (start 145.1686 107.4067) (end 144.9517 107.1898) (width 0.3) (layer F.Cu) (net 1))
 (segment (start 145.85 112.4847) (end 145.1196 112.4847) (width 0.3) (layer F.Cu) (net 1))
 (segment (start 148.7998 107.5881) (end 147.7497 107.5881) (width 0.3) (layer F.Cu) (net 1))
 (segment (start 144.9517 106.44) (end 144.9517 107.1898) (width 0.3) (layer F.Cu) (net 1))
 (segment (start 145.85 113.21) (end 145.85 112.4847) (width 0.3) (layer F.Cu) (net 1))
 (segment (start 141.92 111.42) (end 143.7943 111.42) (width 0.3) (layer B.Cu) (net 1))
 (via (at 145.1686 108.1958) (size 0.8) (layers F.Cu B.Cu) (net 1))
 (via (at 145.1196 112.4847) (size 0.8) (layers F.Cu B.Cu) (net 1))
 (segment (start 146.34 106.44) (end 144.95168 106.44) (width 0.3) (layer F.Cu) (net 1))
 (segment (start 148.79978 107.58808) (end 147.48808 107.58808) (width 0.3) (layer F.Cu) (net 1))
 (segment (start 147.48808 107.58808) (end 146.34 106.44) (width 0.3) (layer F.Cu) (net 1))
 (segment (start 149.8499 105.2919) (end 150.678 106.12) (width 0.3) (layer F.Cu) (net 2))
 (segment (start 150.678 106.12) (end 150.6922 106.12) (width 0.3) (layer F.Cu) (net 2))
 (segment (start 147.7497 105.2919) (end 149.8499 105.2919) (width 0.3) (layer F.Cu) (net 2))
 (segment (start 147.1578 104.7) (end 147.7497 105.2919) (width 0.3) (layer F.Cu) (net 2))
 (segment (start 143.86 104.7) (end 147.1578 104.7) (width 0.3) (layer F.Cu) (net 2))
 (segment (start 145.58 111.31) (end 144.36 110.09) (width 0.3) (layer F.Cu) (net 2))
 (segment (start 144.36 110.09) (end 144.36 108.403998) (width 0.3) (layer F.Cu) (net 2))
 (segment (start 144.36 108.403998) (end 143.64 107.683998) (width 0.3) (layer F.Cu) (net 2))
 (segment (start 145.85 111.31) (end 145.58 111.31) (width 0.3) (layer F.Cu) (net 2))
 (segment (start 143.64 107.683998) (end 143.64 104.92) (width 0.3) (layer F.Cu) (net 2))
 (segment (start 143.64 104.92) (end 143.86 104.7) (width 0.3) (layer F.Cu) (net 2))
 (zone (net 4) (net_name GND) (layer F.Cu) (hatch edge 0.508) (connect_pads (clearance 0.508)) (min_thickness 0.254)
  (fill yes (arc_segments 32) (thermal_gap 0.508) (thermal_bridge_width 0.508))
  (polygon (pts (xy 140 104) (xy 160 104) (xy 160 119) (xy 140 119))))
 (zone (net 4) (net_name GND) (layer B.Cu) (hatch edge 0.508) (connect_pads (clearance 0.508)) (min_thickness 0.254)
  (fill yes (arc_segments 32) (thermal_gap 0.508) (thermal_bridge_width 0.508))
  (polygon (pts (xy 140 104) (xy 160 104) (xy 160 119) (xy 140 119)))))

